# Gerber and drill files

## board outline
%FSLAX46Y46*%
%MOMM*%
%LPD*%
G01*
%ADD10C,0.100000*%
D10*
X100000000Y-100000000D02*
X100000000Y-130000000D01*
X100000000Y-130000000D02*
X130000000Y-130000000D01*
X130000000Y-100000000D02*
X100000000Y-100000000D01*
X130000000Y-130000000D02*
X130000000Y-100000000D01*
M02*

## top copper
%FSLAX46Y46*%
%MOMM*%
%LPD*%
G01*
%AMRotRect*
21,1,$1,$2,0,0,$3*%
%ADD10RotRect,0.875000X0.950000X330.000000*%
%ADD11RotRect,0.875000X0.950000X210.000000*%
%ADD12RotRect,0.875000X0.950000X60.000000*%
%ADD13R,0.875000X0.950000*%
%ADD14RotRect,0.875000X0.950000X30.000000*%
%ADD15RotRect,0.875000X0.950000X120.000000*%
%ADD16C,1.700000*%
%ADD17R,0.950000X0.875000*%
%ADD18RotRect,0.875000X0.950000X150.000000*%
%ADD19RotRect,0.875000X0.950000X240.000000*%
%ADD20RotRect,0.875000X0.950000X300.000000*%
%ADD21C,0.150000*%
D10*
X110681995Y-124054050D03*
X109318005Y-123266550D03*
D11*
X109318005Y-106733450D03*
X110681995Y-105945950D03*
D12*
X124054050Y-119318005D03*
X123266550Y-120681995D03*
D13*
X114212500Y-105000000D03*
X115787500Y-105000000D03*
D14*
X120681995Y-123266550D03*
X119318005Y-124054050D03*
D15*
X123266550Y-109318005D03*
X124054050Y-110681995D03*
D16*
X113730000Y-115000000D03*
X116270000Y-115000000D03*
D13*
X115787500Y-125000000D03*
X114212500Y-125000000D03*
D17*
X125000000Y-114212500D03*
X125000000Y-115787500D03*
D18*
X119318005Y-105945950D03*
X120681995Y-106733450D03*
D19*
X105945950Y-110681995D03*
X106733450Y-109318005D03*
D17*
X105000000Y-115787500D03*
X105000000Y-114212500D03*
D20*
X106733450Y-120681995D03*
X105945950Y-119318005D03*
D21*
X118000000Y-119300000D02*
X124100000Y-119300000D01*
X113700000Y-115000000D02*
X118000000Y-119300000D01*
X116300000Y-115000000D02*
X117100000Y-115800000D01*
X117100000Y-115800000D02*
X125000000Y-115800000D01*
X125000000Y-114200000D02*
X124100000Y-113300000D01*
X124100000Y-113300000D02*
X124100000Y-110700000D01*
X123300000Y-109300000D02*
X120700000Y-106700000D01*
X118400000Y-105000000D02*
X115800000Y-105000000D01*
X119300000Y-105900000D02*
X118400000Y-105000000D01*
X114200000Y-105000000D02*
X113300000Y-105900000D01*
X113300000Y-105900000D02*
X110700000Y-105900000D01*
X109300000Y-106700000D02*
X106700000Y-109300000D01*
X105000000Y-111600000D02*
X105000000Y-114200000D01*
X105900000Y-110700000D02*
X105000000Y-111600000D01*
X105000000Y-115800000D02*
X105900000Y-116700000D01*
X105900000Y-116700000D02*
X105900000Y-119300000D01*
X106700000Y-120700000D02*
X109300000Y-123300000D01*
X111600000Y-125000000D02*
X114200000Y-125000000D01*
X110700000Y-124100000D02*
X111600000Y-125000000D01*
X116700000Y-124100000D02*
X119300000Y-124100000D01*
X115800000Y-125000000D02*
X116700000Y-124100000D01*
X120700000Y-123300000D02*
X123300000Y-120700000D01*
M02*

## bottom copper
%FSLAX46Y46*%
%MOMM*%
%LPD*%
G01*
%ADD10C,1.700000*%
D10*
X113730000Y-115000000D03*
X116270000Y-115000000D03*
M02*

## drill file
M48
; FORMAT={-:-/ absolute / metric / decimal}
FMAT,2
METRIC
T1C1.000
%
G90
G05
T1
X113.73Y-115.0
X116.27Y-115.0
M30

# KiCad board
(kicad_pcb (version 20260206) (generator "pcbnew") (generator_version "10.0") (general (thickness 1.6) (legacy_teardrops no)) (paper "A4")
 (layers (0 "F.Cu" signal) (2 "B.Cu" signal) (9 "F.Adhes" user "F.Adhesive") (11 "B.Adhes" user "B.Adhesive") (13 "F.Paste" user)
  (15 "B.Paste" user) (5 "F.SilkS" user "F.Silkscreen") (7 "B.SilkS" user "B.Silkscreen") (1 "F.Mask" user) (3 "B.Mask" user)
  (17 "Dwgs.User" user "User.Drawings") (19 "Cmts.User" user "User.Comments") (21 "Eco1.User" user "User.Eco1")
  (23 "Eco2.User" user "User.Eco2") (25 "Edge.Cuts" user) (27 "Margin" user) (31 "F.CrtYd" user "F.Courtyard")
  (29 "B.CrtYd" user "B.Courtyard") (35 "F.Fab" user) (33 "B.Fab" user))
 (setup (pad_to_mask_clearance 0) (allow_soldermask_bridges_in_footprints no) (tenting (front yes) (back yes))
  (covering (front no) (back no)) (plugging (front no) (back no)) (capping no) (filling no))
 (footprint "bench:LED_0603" (layer "F.Cu") (at 110 123.6603 -30)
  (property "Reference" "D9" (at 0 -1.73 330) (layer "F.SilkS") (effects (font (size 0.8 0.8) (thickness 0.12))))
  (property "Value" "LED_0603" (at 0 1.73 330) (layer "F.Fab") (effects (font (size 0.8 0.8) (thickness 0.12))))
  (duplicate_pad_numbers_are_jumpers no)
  (pad "A" smd rect (at 0.7875 0 330) (size 0.875 0.95) (layers "F.Cu" "F.Mask" "F.Paste") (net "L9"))
  (pad "K" smd rect (at -0.7875 0 330) (size 0.875 0.95) (layers "F.Cu" "F.Mask" "F.Paste") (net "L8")))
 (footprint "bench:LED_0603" (layer "F.Cu") (at 110 106.3397 -150)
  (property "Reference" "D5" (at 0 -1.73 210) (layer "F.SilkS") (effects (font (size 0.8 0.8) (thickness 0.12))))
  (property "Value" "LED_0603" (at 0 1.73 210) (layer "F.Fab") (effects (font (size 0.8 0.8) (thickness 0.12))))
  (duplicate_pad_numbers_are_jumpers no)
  (pad "A" smd rect (at 0.7875 0 210) (size 0.875 0.95) (layers "F.Cu" "F.Mask" "F.Paste") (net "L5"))
  (pad "K" smd rect (at -0.7875 0 210) (size 0.875 0.95) (layers "F.Cu" "F.Mask" "F.Paste") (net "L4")))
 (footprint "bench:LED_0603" (layer "F.Cu") (at 123.6603 120 60)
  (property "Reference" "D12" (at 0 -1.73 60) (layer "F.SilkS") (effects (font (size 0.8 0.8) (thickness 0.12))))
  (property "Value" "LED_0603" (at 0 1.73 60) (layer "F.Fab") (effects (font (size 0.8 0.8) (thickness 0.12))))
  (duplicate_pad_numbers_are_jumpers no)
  (pad "A" smd rect (at 0.7875 0 60) (size 0.875 0.95) (layers "F.Cu" "F.Mask" "F.Paste") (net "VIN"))
  (pad "K" smd rect (at -0.7875 0 60) (size 0.875 0.95) (layers "F.Cu" "F.Mask" "F.Paste") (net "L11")))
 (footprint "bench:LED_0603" (layer "F.Cu") (at 115 105 180)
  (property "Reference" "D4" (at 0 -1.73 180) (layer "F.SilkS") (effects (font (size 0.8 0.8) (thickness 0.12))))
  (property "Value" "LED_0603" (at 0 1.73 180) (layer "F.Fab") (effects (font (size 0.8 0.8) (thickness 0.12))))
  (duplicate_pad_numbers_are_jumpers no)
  (pad "A" smd rect (at 0.7875 0 180) (size 0.875 0.95) (layers "F.Cu" "F.Mask" "F.Paste") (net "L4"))
  (pad "K" smd rect (at -0.7875 0 180) (size 0.875 0.95) (layers "F.Cu" "F.Mask" "F.Paste") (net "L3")))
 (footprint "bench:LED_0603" (layer "F.Cu") (at 120 123.6603 30)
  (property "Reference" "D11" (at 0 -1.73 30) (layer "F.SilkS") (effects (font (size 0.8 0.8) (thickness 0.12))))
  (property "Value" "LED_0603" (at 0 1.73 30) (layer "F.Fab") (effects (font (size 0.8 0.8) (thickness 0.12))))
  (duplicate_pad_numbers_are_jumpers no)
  (pad "A" smd rect (at 0.7875 0 30) (size 0.875 0.95) (layers "F.Cu" "F.Mask" "F.Paste") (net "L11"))
  (pad "K" smd rect (at -0.7875 0 30) (size 0.875 0.95) (layers "F.Cu" "F.Mask" "F.Paste") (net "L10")))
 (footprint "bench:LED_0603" (layer "F.Cu") (at 123.6603 110 120)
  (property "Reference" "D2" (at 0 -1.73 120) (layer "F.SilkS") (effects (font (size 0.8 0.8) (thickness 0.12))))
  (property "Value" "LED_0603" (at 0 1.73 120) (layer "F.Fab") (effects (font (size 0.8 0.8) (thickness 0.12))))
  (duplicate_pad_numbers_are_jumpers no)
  (pad "A" smd rect (at 0.7875 0 120) (size 0.875 0.95) (layers "F.Cu" "F.Mask" "F.Paste") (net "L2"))
  (pad "K" smd rect (at -0.7875 0 120) (size 0.875 0.95) (layers "F.Cu" "F.Mask" "F.Paste") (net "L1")))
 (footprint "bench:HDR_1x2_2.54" (layer "F.Cu") (at 113.73 115)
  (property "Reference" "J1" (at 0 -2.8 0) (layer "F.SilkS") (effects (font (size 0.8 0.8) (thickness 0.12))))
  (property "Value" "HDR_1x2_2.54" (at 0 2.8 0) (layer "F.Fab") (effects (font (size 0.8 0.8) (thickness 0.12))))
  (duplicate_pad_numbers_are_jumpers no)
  (pad "1" thru_hole circle (at 0 0) (size 1.7 1.7) (drill 1) (layers "*.Cu" "*.Mask") (remove_unused_layers no) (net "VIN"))
  (pad "2" thru_hole circle (at 2.54 0) (size 1.7 1.7) (drill 1) (layers "*.Cu" "*.Mask") (remove_unused_layers no) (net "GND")))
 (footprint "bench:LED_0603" (layer "F.Cu") (at 115 125)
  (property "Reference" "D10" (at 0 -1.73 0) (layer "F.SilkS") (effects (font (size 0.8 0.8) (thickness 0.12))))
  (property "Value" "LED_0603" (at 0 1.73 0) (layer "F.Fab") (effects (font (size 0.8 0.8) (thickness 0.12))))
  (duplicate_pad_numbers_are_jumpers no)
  (pad "A" smd rect (at 0.7875 0) (size 0.875 0.95) (layers "F.Cu" "F.Mask" "F.Paste") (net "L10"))
  (pad "K" smd rect (at -0.7875 0) (size 0.875 0.95) (layers "F.Cu" "F.Mask" "F.Paste") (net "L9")))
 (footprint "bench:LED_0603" (layer "F.Cu") (at 125 115 90)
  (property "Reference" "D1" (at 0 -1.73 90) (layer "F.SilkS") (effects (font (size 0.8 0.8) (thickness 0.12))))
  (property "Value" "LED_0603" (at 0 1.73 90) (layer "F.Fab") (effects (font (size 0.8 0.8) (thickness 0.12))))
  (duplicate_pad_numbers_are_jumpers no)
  (pad "A" smd rect (at 0.7875 0 90) (size 0.875 0.95) (layers "F.Cu" "F.Mask" "F.Paste") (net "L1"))
  (pad "K" smd rect (at -0.7875 0 90) (size 0.875 0.95) (layers "F.Cu" "F.Mask" "F.Paste") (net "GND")))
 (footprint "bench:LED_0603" (layer "F.Cu") (at 120 106.3397 150)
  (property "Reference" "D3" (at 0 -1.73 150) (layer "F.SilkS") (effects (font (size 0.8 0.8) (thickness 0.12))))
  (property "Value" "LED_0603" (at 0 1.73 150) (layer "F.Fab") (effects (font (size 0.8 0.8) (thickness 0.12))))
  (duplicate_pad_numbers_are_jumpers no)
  (pad "A" smd rect (at 0.7875 0 150) (size 0.875 0.95) (layers "F.Cu" "F.Mask" "F.Paste") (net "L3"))
  (pad "K" smd rect (at -0.7875 0 150) (size 0.875 0.95) (layers "F.Cu" "F.Mask" "F.Paste") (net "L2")))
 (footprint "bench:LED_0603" (layer "F.Cu") (at 106.3397 110 -120)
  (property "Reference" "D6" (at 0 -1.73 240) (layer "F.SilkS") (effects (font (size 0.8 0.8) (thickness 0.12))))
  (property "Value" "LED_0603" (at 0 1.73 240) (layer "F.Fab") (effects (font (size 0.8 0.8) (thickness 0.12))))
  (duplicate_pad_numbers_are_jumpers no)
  (pad "A" smd rect (at 0.7875 0 240) (size 0.875 0.95) (layers "F.Cu" "F.Mask" "F.Paste") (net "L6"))
  (pad "K" smd rect (at -0.7875 0 240) (size 0.875 0.95) (layers "F.Cu" "F.Mask" "F.Paste") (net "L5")))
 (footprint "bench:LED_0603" (layer "F.Cu") (at 105 115 -90)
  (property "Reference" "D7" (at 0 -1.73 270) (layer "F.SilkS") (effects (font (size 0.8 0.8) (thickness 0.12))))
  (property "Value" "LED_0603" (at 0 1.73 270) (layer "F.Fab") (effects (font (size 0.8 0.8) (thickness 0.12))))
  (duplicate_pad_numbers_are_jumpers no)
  (pad "A" smd rect (at 0.7875 0 270) (size 0.875 0.95) (layers "F.Cu" "F.Mask" "F.Paste") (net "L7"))
  (pad "K" smd rect (at -0.7875 0 270) (size 0.875 0.95) (layers "F.Cu" "F.Mask" "F.Paste") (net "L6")))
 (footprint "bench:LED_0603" (layer "F.Cu") (at 106.3397 120 -60)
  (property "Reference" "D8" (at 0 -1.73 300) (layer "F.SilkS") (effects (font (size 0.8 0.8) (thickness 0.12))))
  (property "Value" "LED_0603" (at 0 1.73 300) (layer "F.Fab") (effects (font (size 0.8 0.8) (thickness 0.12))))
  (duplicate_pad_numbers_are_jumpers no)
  (pad "A" smd rect (at 0.7875 0 300) (size 0.875 0.95) (layers "F.Cu" "F.Mask" "F.Paste") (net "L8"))
  (pad "K" smd rect (at -0.7875 0 300) (size 0.875 0.95) (layers "F.Cu" "F.Mask" "F.Paste") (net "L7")))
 (gr_line (start 100 100) (end 100 130) (stroke (width 0.1) (type solid)) (layer "Edge.Cuts"))
 (gr_line (start 100 130) (end 130 130) (stroke (width 0.1) (type solid)) (layer "Edge.Cuts"))
 (gr_line (start 130 100) (end 100 100) (stroke (width 0.1) (type solid)) (layer "Edge.Cuts"))
 (gr_line (start 130 130) (end 130 100) (stroke (width 0.1) (type solid)) (layer "Edge.Cuts"))
 (segment (start 118 119.3) (end 124.1 119.3) (width 0.15) (layer "F.Cu") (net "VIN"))
 (segment (start 113.7 115) (end 118 119.3) (width 0.15) (layer "F.Cu") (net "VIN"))
 (segment (start 116.3 115) (end 117.1 115.8) (width 0.15) (layer "F.Cu") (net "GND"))
 (segment (start 117.1 115.8) (end 125 115.8) (width 0.15) (layer "F.Cu") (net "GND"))
 (segment (start 125 114.2) (end 124.1 113.3) (width 0.15) (layer "F.Cu") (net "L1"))
 (segment (start 124.1 113.3) (end 124.1 110.7) (width 0.15) (layer "F.Cu") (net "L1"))
 (segment (start 123.3 109.3) (end 120.7 106.7) (width 0.15) (layer "F.Cu") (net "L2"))
 (segment (start 118.4 105) (end 115.8 105) (width 0.15) (layer "F.Cu") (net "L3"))
 (segment (start 119.3 105.9) (end 118.4 105) (width 0.15) (layer "F.Cu") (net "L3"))
 (segment (start 114.2 105) (end 113.3 105.9) (width 0.15) (layer "F.Cu") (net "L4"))
 (segment (start 113.3 105.9) (end 110.7 105.9) (width 0.15) (layer "F.Cu") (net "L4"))
 (segment (start 109.3 106.7) (end 106.7 109.3) (width 0.15) (layer "F.Cu") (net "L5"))
 (segment (start 105 111.6) (end 105 114.2) (width 0.15) (layer "F.Cu") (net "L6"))
 (segment (start 105.9 110.7) (end 105 111.6) (width 0.15) (layer "F.Cu") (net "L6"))
 (segment (start 105 115.8) (end 105.9 116.7) (width 0.15) (layer "F.Cu") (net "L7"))
 (segment (start 105.9 116.7) (end 105.9 119.3) (width 0.15) (layer "F.Cu") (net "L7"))
 (segment (start 106.7 120.7) (end 109.3 123.3) (width 0.15) (layer "F.Cu") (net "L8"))
 (segment (start 111.6 125) (end 114.2 125) (width 0.15) (layer "F.Cu") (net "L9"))
 (segment (start 110.7 124.1) (end 111.6 125) (width 0.15) (layer "F.Cu") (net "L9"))
 (segment (start 116.7 124.1) (end 119.3 124.1) (width 0.15) (layer "F.Cu") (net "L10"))
 (segment (start 115.8 125) (end 116.7 124.1) (width 0.15) (layer "F.Cu") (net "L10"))
 (segment (start 120.7 123.3) (end 123.3 120.7) (width 0.15) (layer "F.Cu") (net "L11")))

